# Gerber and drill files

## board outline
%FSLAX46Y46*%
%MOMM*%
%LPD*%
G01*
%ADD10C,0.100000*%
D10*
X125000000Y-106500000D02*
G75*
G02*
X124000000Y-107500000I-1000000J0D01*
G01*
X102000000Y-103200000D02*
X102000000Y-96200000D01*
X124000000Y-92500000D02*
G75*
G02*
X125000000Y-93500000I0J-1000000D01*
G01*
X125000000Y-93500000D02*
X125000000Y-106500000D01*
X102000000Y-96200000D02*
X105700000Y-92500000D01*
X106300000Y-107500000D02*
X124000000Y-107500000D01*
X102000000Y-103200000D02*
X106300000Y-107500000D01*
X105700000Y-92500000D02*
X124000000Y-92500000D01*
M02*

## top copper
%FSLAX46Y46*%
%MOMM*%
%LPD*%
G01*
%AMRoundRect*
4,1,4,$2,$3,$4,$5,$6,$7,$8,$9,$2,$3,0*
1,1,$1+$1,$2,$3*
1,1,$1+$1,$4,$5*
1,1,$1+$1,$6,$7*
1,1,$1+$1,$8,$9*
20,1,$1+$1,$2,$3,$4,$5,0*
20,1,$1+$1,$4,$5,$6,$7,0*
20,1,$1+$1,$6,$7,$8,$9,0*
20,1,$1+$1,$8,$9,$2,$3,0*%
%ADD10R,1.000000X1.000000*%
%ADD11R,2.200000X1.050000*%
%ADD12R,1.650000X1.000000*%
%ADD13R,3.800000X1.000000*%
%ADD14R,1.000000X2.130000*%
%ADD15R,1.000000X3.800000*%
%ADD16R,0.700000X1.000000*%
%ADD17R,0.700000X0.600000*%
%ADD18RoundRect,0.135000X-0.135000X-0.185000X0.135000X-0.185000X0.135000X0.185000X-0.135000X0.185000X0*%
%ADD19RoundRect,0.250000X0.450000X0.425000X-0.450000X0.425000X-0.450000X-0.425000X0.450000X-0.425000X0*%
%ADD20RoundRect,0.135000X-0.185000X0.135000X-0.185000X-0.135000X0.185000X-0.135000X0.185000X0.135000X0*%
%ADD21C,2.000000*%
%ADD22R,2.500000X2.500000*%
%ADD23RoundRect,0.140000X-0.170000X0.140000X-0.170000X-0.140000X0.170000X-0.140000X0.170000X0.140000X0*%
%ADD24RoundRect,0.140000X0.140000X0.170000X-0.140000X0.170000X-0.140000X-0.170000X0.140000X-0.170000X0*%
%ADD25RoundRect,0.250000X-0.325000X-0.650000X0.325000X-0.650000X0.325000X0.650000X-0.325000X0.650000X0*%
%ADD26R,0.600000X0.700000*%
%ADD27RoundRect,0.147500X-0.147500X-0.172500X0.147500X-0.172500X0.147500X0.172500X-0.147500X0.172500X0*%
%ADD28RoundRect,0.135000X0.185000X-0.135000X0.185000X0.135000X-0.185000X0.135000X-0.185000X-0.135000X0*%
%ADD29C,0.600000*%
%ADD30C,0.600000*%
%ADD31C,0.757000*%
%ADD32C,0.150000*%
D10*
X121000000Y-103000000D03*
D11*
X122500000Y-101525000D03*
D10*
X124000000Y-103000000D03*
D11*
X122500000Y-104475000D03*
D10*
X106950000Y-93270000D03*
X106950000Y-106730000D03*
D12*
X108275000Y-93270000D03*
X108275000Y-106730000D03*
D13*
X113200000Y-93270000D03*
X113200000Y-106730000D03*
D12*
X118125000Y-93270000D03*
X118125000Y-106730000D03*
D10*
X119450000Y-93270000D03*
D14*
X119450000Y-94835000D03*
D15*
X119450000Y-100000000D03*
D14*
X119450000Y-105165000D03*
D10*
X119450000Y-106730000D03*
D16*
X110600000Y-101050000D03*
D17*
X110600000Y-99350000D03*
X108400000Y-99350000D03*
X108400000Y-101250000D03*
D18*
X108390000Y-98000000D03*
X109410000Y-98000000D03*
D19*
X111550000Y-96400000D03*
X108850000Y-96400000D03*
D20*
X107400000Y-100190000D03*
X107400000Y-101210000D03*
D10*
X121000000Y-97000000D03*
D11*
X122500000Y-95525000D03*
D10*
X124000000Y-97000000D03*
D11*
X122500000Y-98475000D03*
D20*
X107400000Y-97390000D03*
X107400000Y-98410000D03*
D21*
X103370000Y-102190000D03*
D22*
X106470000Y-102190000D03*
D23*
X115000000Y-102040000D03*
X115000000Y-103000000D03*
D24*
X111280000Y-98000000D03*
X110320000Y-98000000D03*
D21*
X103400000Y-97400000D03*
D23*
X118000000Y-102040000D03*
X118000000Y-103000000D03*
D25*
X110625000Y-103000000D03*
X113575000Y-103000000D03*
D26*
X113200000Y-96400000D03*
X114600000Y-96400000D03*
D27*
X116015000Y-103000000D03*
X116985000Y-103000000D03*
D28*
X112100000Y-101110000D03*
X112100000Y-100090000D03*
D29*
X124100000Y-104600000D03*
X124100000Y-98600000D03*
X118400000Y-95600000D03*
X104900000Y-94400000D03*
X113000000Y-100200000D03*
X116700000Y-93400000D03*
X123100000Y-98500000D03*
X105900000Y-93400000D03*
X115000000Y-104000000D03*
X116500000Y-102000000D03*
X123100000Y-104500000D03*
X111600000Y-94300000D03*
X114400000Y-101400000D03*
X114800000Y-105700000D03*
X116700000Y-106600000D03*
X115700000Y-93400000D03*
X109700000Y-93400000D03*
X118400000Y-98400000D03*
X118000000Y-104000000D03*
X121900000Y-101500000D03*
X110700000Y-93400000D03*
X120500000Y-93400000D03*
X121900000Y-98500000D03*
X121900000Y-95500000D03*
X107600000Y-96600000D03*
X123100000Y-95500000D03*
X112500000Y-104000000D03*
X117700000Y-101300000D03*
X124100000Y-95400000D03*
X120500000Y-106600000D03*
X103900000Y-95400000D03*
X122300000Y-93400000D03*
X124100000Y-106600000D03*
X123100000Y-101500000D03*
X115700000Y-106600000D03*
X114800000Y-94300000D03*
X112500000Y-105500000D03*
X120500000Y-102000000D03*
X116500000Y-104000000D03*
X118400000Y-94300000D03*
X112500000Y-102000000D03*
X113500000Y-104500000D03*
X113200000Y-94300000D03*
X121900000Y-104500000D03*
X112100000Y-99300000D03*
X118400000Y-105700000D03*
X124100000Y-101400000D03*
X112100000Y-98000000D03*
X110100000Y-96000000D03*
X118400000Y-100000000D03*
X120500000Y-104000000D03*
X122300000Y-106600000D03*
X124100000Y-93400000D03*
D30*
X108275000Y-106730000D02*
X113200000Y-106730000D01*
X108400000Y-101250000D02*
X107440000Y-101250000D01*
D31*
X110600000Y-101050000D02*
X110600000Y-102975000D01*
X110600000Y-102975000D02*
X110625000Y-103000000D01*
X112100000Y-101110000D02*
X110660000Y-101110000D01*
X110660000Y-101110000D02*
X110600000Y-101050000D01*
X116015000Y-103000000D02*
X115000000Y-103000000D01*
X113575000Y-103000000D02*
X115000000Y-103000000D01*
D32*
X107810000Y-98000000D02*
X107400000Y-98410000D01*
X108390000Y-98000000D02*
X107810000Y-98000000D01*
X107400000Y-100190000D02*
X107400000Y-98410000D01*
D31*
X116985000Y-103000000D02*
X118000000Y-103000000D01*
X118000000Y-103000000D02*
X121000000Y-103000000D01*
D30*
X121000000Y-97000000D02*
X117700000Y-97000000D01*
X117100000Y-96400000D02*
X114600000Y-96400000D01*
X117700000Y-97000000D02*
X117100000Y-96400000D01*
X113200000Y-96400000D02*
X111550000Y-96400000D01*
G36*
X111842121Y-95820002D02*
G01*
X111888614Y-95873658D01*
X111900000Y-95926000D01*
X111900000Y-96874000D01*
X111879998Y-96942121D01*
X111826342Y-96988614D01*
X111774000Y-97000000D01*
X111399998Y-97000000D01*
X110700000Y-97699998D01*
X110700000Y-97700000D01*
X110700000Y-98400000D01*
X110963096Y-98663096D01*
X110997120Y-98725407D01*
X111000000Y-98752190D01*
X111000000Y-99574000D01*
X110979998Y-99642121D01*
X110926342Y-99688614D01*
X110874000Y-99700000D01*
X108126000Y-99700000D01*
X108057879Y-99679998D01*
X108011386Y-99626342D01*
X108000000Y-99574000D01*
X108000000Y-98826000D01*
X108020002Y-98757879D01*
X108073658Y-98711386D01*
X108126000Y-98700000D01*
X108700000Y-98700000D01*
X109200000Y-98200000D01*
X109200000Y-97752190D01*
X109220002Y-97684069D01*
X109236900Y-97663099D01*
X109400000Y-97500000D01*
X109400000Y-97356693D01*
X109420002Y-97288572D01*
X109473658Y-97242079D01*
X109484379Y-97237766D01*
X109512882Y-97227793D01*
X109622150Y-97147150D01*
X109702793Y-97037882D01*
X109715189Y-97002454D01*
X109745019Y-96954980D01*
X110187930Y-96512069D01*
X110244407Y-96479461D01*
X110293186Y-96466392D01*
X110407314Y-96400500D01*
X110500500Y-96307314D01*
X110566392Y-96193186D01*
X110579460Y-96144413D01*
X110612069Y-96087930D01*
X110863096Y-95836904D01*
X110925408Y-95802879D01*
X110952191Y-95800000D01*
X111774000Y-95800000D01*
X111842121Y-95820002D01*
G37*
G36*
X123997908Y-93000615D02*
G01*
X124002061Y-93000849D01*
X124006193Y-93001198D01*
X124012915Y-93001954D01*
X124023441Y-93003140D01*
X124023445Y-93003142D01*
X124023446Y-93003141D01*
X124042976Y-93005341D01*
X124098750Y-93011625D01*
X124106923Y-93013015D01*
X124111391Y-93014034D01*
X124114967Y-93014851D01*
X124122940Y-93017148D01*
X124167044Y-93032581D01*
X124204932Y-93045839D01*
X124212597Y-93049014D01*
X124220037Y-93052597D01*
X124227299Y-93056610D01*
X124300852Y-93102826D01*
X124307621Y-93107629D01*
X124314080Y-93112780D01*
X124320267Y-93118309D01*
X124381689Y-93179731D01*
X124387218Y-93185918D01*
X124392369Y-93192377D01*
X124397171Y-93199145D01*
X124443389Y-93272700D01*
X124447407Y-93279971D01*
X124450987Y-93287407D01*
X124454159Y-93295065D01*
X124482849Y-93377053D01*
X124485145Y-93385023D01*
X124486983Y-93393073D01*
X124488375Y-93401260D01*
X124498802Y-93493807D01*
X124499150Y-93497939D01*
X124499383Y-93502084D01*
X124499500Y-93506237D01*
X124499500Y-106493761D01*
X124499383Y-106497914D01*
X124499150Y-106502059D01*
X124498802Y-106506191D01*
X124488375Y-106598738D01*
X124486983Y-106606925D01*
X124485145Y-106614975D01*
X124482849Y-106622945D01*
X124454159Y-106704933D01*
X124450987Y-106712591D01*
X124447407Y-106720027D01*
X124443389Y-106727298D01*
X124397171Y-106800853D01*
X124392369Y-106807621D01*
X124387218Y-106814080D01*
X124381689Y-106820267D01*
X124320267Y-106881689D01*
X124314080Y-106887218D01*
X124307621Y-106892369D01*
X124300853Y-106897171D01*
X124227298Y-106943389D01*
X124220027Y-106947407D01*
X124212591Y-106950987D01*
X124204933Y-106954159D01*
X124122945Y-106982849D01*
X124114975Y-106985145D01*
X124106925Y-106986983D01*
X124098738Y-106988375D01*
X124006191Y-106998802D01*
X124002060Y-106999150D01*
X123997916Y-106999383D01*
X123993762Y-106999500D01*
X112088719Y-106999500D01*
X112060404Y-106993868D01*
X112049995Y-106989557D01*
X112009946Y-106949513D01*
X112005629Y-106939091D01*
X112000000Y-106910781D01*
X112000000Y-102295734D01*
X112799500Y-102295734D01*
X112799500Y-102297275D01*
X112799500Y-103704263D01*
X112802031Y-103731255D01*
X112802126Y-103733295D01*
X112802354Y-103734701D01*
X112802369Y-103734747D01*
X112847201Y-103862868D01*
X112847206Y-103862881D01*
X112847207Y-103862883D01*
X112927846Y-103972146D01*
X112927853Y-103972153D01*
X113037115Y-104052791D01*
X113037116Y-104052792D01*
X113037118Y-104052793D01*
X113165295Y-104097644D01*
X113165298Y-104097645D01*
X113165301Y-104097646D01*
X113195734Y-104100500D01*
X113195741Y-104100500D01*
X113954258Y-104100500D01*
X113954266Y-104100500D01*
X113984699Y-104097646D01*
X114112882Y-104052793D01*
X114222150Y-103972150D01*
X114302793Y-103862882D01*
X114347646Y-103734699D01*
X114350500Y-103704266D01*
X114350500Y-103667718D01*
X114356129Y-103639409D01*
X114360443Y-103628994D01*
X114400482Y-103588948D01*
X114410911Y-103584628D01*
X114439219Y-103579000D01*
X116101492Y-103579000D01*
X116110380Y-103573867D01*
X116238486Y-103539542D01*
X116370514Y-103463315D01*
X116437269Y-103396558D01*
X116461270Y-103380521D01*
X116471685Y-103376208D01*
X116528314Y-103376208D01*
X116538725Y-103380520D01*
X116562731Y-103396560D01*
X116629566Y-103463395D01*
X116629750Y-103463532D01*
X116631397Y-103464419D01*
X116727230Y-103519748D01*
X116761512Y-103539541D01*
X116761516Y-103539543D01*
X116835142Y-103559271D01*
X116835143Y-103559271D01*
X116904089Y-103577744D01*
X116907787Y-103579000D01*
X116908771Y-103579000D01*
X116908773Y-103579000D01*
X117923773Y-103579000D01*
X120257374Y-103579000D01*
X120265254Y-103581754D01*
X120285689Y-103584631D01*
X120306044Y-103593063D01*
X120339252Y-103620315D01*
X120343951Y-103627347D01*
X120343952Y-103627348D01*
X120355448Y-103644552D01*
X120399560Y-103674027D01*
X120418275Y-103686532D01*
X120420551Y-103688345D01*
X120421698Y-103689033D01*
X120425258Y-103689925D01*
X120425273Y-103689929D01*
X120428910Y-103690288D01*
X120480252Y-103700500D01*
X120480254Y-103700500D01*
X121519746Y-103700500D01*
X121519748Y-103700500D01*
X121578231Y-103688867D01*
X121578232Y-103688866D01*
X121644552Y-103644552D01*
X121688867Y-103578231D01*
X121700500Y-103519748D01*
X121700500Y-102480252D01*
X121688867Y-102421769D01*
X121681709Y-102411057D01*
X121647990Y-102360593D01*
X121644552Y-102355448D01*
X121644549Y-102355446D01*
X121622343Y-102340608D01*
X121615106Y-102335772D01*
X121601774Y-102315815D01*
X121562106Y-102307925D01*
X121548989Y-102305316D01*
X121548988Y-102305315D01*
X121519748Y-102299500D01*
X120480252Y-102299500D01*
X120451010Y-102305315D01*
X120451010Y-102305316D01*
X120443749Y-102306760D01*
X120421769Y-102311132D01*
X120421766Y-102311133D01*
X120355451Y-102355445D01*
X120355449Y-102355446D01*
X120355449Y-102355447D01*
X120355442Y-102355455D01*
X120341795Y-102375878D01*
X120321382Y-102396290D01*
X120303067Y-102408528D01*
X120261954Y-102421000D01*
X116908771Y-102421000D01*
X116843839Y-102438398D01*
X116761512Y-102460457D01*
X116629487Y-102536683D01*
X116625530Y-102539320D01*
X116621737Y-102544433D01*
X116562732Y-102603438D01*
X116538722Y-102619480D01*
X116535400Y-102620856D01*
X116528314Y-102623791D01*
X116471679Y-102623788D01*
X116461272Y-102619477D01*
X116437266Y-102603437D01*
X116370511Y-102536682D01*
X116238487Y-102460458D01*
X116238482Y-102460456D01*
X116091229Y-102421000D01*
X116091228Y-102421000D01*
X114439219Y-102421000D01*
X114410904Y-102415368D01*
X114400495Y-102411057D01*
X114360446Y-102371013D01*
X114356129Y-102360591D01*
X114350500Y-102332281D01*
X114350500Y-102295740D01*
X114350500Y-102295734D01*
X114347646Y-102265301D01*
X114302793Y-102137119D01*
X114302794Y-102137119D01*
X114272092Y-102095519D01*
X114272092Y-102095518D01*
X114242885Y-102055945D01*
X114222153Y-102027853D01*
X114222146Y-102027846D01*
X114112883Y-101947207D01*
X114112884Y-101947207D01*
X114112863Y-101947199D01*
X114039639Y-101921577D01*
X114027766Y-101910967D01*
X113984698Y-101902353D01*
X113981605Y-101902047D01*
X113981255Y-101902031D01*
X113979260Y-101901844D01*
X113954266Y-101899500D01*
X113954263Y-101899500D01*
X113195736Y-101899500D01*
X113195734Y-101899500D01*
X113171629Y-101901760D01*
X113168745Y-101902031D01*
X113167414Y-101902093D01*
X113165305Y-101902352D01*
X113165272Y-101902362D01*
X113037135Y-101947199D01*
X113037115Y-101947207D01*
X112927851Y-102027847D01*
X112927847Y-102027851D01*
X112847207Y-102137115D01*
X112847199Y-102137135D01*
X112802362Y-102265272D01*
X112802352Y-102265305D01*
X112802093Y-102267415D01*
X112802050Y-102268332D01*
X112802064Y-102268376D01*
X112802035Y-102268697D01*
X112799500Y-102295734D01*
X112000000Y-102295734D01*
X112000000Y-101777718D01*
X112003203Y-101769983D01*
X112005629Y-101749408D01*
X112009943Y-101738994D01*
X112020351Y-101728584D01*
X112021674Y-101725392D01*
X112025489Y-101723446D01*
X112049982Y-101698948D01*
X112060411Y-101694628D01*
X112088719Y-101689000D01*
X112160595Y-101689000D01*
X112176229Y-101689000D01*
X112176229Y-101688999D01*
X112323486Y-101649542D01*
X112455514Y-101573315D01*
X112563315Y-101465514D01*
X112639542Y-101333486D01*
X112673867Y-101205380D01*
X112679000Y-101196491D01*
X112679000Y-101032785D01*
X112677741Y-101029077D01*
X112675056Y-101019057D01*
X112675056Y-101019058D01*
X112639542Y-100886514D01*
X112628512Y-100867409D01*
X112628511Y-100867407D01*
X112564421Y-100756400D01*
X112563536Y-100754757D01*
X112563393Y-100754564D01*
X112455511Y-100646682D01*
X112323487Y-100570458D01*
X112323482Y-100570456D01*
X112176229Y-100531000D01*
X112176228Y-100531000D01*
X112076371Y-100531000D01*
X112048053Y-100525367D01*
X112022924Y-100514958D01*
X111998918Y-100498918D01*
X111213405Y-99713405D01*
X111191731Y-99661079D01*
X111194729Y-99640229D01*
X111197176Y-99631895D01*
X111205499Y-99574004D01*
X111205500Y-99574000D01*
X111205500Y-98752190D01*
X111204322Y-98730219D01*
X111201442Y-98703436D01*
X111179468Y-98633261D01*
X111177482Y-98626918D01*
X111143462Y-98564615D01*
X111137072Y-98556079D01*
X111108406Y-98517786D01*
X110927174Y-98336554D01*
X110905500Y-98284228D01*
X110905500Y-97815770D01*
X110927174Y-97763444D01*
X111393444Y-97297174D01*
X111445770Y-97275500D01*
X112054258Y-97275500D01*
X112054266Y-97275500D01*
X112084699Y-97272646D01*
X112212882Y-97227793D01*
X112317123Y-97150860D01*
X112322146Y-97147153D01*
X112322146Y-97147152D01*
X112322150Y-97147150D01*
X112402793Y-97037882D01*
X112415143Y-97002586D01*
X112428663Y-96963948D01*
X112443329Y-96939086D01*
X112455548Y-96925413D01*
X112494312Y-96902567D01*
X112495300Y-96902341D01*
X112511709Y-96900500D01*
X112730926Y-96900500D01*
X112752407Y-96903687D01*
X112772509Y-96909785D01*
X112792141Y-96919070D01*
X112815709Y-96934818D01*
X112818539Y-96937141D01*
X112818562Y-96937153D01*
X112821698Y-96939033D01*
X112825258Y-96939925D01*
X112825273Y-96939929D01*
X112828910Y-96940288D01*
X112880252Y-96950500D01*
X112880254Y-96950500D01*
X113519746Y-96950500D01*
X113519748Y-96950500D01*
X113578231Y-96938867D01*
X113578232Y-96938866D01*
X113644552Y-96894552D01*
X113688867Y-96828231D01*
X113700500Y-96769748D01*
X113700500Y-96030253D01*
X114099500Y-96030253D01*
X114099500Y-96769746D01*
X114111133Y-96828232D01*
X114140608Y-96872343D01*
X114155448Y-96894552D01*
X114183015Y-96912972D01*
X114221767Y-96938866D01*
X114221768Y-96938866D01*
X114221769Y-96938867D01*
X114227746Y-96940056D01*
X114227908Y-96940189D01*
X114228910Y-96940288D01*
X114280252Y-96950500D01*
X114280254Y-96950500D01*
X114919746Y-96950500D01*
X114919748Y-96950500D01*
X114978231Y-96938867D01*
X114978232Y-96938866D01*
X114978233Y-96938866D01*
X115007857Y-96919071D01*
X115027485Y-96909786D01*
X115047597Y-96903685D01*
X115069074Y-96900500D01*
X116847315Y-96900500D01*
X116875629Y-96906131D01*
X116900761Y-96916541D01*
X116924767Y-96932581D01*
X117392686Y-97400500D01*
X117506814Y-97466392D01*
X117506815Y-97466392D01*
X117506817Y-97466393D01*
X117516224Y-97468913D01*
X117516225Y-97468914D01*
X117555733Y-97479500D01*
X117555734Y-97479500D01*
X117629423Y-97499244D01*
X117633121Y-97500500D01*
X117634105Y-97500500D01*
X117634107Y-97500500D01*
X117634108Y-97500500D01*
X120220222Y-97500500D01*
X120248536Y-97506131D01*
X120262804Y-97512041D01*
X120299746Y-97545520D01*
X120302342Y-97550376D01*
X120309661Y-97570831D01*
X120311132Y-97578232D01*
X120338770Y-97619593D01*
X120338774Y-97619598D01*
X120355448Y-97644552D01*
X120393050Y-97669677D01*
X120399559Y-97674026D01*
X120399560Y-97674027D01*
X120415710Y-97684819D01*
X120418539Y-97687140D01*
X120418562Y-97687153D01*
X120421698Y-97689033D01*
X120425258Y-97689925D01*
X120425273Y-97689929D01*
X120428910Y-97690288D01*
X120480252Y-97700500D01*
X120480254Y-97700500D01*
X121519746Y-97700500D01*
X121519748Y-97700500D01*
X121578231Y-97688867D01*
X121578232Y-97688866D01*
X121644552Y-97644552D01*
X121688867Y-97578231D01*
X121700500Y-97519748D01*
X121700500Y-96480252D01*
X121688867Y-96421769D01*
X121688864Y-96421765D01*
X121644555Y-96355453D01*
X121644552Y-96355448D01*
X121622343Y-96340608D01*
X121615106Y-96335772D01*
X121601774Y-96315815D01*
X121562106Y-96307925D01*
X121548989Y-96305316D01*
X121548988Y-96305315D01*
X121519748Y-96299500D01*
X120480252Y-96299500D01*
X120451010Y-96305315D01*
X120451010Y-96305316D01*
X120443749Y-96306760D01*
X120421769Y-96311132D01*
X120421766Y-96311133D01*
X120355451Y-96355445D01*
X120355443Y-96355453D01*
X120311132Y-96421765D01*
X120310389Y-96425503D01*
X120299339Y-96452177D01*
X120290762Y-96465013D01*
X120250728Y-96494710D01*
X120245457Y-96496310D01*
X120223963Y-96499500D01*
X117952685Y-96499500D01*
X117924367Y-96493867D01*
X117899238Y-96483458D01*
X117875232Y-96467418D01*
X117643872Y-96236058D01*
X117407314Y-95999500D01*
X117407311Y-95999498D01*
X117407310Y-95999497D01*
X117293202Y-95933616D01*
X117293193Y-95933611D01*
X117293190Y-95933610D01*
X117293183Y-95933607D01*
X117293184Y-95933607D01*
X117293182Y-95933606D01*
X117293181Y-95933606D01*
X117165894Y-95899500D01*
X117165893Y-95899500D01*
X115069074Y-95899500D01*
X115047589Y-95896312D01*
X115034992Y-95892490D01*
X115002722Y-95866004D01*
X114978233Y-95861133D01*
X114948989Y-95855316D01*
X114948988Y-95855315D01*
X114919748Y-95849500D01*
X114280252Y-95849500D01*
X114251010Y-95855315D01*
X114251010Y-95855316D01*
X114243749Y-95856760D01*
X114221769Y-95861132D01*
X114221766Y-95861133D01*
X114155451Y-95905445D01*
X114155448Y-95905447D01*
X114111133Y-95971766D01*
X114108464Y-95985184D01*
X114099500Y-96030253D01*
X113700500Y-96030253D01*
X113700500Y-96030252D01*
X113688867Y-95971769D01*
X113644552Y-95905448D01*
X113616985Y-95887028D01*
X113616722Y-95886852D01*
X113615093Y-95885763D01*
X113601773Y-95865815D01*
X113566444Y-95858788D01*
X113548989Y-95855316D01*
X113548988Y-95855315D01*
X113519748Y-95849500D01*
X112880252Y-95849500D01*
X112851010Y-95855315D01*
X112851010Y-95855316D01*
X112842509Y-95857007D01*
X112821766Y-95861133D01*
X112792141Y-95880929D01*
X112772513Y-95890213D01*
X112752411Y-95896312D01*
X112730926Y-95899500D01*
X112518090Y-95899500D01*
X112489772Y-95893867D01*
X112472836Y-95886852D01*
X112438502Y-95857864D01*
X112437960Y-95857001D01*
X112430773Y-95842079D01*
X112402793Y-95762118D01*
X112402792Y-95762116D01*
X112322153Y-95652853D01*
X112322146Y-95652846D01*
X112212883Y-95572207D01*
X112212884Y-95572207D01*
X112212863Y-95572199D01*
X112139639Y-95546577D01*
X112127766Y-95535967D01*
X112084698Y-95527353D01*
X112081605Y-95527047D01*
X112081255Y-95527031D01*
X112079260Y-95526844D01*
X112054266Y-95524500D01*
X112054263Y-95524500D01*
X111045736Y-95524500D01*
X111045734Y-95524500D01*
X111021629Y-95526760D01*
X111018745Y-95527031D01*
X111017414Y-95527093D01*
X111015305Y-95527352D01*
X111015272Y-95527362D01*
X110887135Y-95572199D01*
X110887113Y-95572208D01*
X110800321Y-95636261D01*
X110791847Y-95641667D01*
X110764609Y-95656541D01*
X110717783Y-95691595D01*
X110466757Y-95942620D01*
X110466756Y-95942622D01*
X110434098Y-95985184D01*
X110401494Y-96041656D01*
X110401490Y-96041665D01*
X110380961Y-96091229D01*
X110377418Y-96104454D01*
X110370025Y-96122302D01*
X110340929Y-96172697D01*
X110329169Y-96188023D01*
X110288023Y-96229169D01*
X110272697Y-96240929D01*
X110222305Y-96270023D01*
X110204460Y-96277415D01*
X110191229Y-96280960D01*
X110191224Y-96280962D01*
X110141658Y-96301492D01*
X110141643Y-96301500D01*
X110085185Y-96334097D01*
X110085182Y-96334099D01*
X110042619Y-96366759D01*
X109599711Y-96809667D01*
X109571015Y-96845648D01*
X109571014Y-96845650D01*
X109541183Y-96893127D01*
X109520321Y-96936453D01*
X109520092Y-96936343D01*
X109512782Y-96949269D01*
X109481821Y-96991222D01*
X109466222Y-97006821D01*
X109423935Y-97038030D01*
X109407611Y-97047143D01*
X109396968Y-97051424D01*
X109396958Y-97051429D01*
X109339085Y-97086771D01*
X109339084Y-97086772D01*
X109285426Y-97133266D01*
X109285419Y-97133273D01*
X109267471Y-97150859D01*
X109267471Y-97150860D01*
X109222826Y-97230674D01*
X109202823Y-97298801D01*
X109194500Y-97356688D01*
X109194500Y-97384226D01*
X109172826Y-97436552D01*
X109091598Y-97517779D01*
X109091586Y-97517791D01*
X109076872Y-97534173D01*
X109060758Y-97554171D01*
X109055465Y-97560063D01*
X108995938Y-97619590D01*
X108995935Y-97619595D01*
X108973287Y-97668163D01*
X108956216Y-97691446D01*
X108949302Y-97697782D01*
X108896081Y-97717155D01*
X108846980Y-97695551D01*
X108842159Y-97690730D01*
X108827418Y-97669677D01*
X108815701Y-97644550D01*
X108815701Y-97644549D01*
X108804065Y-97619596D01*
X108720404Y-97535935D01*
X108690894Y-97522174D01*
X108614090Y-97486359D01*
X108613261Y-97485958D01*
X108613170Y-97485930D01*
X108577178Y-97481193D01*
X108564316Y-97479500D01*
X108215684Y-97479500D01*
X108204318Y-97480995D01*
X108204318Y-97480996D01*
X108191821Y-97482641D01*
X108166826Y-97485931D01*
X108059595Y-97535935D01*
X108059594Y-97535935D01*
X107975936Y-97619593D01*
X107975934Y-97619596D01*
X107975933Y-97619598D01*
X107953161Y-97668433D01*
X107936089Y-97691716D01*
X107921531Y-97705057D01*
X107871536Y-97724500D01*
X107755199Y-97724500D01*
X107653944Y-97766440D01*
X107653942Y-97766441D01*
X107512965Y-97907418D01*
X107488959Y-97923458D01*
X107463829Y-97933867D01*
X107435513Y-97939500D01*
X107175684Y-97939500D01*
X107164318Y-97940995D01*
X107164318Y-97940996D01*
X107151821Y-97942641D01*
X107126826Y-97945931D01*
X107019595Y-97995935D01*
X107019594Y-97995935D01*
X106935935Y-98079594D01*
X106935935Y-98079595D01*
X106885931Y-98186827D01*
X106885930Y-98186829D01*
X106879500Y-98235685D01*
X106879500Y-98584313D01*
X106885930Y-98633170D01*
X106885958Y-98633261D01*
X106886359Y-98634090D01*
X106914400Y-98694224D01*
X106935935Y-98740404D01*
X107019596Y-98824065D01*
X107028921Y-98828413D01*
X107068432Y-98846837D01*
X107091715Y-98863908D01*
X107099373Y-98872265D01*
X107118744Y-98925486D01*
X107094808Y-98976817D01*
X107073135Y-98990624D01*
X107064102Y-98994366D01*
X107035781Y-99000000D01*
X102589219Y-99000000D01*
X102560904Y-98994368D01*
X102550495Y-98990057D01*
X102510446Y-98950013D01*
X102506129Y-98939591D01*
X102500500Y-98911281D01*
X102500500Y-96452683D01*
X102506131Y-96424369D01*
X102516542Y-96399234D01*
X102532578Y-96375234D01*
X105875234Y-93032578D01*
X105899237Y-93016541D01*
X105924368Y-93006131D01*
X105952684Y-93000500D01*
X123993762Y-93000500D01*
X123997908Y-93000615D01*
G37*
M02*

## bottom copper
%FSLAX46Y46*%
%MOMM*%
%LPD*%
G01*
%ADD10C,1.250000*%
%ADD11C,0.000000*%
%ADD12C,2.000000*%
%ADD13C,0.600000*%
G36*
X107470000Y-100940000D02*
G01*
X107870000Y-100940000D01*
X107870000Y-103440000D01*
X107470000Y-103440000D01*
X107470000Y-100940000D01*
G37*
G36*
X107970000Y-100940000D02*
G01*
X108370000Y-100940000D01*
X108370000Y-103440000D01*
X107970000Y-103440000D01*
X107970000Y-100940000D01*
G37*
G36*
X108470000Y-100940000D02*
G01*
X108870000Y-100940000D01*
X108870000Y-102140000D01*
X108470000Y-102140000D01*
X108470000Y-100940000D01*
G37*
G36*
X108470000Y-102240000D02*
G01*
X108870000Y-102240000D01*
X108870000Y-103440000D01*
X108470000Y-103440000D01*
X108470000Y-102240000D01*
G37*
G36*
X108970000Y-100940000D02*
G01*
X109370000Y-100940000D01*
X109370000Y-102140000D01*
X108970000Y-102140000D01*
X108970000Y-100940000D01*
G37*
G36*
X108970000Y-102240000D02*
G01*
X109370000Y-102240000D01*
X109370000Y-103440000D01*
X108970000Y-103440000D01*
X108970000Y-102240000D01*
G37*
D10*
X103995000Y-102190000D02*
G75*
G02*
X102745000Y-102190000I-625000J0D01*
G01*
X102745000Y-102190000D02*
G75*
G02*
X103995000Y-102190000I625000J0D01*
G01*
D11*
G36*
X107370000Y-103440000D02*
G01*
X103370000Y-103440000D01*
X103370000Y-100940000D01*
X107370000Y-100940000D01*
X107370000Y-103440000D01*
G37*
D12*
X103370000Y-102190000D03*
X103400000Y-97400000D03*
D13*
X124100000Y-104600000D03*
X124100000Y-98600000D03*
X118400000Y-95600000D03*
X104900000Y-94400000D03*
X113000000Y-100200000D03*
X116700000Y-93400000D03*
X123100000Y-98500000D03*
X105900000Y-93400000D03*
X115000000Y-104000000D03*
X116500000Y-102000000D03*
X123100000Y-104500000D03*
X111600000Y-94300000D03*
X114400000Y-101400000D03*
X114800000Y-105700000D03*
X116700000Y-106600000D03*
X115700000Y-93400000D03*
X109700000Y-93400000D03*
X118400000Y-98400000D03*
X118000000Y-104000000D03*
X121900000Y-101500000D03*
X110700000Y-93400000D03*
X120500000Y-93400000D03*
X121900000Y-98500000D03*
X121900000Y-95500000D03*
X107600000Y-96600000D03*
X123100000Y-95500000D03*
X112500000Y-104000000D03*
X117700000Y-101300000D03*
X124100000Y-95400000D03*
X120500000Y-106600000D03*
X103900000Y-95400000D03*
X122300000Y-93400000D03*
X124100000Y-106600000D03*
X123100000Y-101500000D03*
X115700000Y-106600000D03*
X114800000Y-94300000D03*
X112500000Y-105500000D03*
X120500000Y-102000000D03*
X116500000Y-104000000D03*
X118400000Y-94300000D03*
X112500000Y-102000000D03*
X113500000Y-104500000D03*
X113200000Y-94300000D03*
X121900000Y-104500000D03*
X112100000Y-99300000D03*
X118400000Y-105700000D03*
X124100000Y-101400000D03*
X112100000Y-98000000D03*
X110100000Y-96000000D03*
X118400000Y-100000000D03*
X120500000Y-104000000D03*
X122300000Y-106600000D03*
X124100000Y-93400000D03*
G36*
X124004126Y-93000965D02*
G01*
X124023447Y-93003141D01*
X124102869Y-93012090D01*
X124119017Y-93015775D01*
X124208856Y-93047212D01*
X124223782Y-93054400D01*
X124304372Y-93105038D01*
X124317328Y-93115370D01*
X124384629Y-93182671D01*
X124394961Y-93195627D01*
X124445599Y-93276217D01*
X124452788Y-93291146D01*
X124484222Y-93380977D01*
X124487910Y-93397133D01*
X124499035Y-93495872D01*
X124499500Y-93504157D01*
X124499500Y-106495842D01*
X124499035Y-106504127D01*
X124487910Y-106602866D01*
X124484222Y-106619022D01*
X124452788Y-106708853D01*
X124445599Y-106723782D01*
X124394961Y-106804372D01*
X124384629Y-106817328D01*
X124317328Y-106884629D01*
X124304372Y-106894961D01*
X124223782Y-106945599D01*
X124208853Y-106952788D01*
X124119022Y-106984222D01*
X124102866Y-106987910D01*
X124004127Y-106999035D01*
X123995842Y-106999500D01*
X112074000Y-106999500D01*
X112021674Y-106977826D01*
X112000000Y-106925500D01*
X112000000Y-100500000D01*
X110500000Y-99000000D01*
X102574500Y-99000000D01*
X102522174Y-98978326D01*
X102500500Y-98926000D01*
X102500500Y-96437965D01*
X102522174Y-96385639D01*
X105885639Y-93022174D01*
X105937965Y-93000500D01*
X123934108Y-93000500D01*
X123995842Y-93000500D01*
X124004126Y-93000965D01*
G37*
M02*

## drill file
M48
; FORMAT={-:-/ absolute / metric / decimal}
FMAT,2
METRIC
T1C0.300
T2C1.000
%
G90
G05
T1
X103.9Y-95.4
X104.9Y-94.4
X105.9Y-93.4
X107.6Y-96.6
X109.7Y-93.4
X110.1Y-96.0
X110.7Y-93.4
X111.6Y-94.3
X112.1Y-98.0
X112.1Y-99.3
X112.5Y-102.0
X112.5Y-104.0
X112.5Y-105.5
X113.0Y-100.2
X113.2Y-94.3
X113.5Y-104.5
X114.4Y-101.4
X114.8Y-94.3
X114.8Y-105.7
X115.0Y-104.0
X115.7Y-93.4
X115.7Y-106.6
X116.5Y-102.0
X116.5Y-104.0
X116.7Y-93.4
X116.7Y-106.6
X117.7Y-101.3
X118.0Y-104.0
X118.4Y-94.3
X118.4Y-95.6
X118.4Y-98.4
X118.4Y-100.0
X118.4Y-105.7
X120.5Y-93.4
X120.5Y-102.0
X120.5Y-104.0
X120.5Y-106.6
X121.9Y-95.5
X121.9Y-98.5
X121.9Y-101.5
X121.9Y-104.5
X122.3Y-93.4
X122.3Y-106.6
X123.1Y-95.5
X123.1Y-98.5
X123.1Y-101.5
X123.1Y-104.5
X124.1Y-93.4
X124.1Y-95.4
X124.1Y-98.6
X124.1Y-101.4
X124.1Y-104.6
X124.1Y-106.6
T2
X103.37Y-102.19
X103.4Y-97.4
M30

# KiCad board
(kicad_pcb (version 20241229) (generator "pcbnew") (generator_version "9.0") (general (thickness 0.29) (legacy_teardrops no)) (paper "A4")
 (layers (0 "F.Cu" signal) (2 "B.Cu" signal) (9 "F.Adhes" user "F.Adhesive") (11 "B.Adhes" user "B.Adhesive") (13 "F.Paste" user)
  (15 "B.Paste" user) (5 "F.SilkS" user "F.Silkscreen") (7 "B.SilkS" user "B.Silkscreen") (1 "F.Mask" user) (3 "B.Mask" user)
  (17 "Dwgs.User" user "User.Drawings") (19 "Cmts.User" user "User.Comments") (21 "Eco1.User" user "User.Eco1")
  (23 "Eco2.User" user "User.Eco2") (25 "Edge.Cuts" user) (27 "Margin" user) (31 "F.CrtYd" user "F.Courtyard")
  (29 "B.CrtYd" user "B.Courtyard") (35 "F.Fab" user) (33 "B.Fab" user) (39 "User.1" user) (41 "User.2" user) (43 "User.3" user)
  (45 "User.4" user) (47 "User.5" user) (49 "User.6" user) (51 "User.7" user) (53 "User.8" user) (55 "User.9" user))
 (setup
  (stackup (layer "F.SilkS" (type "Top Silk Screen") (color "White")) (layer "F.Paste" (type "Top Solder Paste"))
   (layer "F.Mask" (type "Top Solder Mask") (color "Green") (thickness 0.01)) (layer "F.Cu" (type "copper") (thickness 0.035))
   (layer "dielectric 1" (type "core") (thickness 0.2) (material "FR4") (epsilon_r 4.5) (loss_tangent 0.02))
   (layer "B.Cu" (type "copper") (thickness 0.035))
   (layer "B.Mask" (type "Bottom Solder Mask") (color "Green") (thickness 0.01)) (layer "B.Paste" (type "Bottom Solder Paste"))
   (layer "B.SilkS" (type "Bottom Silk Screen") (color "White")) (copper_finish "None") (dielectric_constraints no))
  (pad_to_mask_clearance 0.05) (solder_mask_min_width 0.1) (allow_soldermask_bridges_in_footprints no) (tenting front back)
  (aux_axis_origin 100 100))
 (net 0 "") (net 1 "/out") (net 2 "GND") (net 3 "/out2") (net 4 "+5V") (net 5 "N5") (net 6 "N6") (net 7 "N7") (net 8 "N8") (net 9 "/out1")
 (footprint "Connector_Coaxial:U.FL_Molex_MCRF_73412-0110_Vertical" (layer "F.Cu") (at 122.5 103 -90)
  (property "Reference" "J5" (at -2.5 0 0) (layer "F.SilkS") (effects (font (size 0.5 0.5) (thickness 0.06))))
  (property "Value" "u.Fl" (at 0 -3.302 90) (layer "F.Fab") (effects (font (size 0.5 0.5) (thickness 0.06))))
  (pad "1" smd rect (at 0 1.5 270) (size 1 1) (layers "F.Cu" "F.Mask" "F.Paste") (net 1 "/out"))
  (pad "2" smd rect (at -1.475 0 270) (size 1.05 2.2) (layers "F.Cu" "F.Mask" "F.Paste") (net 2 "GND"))
  (pad "2" smd rect (at 0 -1.5 270) (size 1 1) (layers "F.Cu" "F.Mask" "F.Paste") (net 2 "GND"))
  (pad "2" smd rect (at 1.475 0 270) (size 1.05 2.2) (layers "F.Cu" "F.Mask" "F.Paste") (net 2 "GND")))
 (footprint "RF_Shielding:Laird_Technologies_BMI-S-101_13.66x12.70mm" (layer "F.Cu") (at 113.2 100)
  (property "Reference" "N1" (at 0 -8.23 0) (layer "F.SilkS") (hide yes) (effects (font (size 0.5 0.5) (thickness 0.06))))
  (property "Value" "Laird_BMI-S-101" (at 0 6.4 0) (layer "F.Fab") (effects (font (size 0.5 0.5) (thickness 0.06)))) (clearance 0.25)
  (pad "1" smd rect (at -6.25 -6.73) (size 1 1) (layers "F.Cu" "F.Mask" "F.Paste") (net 2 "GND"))
  (pad "1" smd rect (at -6.25 6.73) (size 1 1) (layers "F.Cu" "F.Mask" "F.Paste") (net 2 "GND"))
  (pad "1" smd rect (at -4.925 -6.73) (size 1.65 1) (layers "F.Cu" "F.Mask" "F.Paste") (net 2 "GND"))
  (pad "1" smd rect (at -4.925 6.73) (size 1.65 1) (layers "F.Cu" "F.Mask" "F.Paste") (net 2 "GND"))
  (pad "1" smd rect (at 0 -6.73) (size 3.8 1) (layers "F.Cu" "F.Mask" "F.Paste") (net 2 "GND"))
  (pad "1" smd rect (at 0 6.73) (size 3.8 1) (layers "F.Cu" "F.Mask" "F.Paste") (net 2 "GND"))
  (pad "1" smd rect (at 4.925 -6.73) (size 1.65 1) (layers "F.Cu" "F.Mask" "F.Paste") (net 2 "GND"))
  (pad "1" smd rect (at 4.925 6.73) (size 1.65 1) (layers "F.Cu" "F.Mask" "F.Paste") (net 2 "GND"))
  (pad "1" smd rect (at 6.25 -6.73) (size 1 1) (layers "F.Cu" "F.Mask" "F.Paste") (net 2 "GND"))
  (pad "1" smd rect (at 6.25 -5.165) (size 1 2.13) (layers "F.Cu" "F.Mask" "F.Paste") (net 2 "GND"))
  (pad "1" smd rect (at 6.25 0) (size 1 3.8) (layers "F.Cu" "F.Mask" "F.Paste") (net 2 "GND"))
  (pad "1" smd rect (at 6.25 5.165) (size 1 2.13) (layers "F.Cu" "F.Mask" "F.Paste") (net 2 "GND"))
  (pad "1" smd rect (at 6.25 6.73) (size 1 1) (layers "F.Cu" "F.Mask" "F.Paste") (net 2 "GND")))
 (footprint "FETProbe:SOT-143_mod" (layer "F.Cu") (at 109.5 100.3 180)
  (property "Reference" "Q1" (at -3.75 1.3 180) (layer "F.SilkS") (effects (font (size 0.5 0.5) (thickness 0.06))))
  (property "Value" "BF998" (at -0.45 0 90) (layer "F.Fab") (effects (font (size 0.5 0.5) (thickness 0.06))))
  (pad "1" smd rect (at -1.1 -0.75 180) (size 0.7 1) (layers "F.Cu" "F.Mask" "F.Paste") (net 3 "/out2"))
  (pad "2" smd rect (at -1.1 0.95 180) (size 0.7 0.6) (layers "F.Cu" "F.Mask" "F.Paste") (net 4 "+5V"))
  (pad "3" smd rect (at 1.1 0.95 180) (size 0.7 0.6) (layers "F.Cu" "F.Mask" "F.Paste") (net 4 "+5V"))
  (pad "4" smd rect (at 1.1 -0.95 180) (size 0.7 0.6) (layers "F.Cu" "F.Mask" "F.Paste") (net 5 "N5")))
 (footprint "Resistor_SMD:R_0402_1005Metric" (layer "F.Cu") (at 108.9 98)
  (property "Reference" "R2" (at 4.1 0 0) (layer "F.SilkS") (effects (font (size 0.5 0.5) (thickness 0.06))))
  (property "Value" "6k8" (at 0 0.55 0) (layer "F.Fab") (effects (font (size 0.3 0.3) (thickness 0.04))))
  (pad "1" smd roundrect (at -0.51 0) (size 0.54 0.64) (layers "F.Cu" "F.Mask" "F.Paste") (roundrect_rratio 0.25) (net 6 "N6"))
  (pad "2" smd roundrect (at 0.51 0) (size 0.54 0.64) (layers "F.Cu" "F.Mask" "F.Paste") (roundrect_rratio 0.25) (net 4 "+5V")))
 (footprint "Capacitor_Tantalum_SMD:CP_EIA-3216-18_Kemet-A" (layer "F.Cu") (at 110.2 96.4 180)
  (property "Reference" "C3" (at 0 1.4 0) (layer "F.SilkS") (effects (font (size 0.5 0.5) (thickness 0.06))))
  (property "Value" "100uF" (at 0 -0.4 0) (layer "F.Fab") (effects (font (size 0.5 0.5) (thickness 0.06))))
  (pad "1" smd roundrect (at -1.35 0 180) (size 1.4 1.35) (layers "F.Cu" "F.Mask" "F.Paste") (roundrect_rratio 0.1851851852) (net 4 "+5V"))
  (pad "2" smd roundrect (at 1.35 0 180) (size 1.4 1.35) (layers "F.Cu" "F.Mask" "F.Paste") (roundrect_rratio 0.1851851852) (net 2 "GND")))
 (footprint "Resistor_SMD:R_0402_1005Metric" (layer "F.Cu") (at 107.4 100.7 -90)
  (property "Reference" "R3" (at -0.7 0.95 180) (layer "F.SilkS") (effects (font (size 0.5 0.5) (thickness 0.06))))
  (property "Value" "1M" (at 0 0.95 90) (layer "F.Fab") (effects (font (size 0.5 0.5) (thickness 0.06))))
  (pad "1" smd roundrect (at -0.51 0 270) (size 0.54 0.64) (layers "F.Cu" "F.Mask" "F.Paste") (roundrect_rratio 0.25) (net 6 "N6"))
  (pad "2" smd roundrect (at 0.51 0 270) (size 0.54 0.64) (layers "F.Cu" "F.Mask" "F.Paste") (roundrect_rratio 0.25) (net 5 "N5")))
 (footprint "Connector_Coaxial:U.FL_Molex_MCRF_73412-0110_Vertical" (layer "F.Cu") (at 122.5 97 -90)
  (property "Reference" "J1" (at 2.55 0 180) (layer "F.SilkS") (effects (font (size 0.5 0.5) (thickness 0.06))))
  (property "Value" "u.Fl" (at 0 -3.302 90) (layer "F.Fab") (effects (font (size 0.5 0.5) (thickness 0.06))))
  (pad "1" smd rect (at 0 1.5 270) (size 1 1) (layers "F.Cu" "F.Mask" "F.Paste") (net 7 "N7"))
  (pad "2" smd rect (at -1.475 0 270) (size 1.05 2.2) (layers "F.Cu" "F.Mask" "F.Paste") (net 2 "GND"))
  (pad "2" smd rect (at 0 -1.5 270) (size 1 1) (layers "F.Cu" "F.Mask" "F.Paste") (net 2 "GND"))
  (pad "2" smd rect (at 1.475 0 270) (size 1.05 2.2) (layers "F.Cu" "F.Mask" "F.Paste") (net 2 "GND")))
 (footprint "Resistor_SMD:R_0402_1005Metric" (layer "F.Cu") (at 107.4 97.9 -90)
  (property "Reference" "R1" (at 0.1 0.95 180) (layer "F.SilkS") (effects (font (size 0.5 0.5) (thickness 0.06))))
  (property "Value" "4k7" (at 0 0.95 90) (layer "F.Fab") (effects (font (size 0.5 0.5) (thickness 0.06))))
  (pad "1" smd roundrect (at -0.51 0 270) (size 0.54 0.64) (layers "F.Cu" "F.Mask" "F.Paste") (roundrect_rratio 0.25) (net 2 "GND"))
  (pad "2" smd roundrect (at 0.51 0 270) (size 0.54 0.64) (layers "F.Cu" "F.Mask" "F.Paste") (roundrect_rratio 0.25) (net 6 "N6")))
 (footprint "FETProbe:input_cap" (layer "F.Cu") (at 108.07 102.19)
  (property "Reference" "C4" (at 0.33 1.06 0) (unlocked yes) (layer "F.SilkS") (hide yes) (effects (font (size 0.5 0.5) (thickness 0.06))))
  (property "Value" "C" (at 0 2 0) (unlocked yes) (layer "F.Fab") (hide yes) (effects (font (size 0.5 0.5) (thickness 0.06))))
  (fp_rect (start -0.6 -1.25) (end -0.2 1.25) (stroke (width 0) (type solid)) (fill yes) (layer "B.Cu"))
  (fp_rect (start -0.1 -1.25) (end 0.3 1.25) (stroke (width 0) (type solid)) (fill yes) (layer "B.Cu"))
  (fp_rect (start 0.4 -1.25) (end 0.8 -0.05) (stroke (width 0) (type solid)) (fill yes) (layer "B.Cu"))
  (fp_rect (start 0.4 0.05) (end 0.8 1.25) (stroke (width 0) (type solid)) (fill yes) (layer "B.Cu"))
  (fp_rect (start 0.9 -1.25) (end 1.3 -0.05) (stroke (width 0) (type solid)) (fill yes) (layer "B.Cu"))
  (fp_rect (start 0.9 0.05) (end 1.3 1.25) (stroke (width 0) (type solid)) (fill yes) (layer "B.Cu"))
  (fp_circle (center -4.7 0) (end -3.45 0) (stroke (width 0) (type solid)) (fill yes) (layer "B.Cu"))
  (fp_poly (pts (xy -4.7 -1.25) (xy -0.7 -1.25) (xy -0.7 1.25) (xy -4.7 1.25)) (stroke (width 0) (type solid)) (fill yes) (layer "B.Cu"))
  (pad "1" thru_hole circle (at -4.7 0) (size 2 2) (drill 1) (layers "*.Cu" "*.Mask") (remove_unused_layers no) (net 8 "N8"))
  (pad "2" smd rect (at -1.6 0) (size 2.5 2.5) (layers "F.Cu") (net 5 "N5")))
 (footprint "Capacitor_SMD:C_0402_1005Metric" (layer "F.Cu") (at 115 102.52 -90)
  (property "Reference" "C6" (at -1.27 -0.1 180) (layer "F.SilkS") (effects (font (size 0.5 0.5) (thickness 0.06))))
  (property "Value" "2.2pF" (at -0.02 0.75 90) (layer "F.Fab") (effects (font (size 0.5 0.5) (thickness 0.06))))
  (pad "1" smd roundrect (at -0.48 0 270) (size 0.56 0.62) (layers "F.Cu" "F.Mask" "F.Paste") (roundrect_rratio 0.25) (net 2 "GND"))
  (pad "2" smd roundrect (at 0.48 0 270) (size 0.56 0.62) (layers "F.Cu" "F.Mask" "F.Paste") (roundrect_rratio 0.25) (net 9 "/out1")))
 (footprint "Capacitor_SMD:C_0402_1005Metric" (layer "F.Cu") (at 110.8 98 180)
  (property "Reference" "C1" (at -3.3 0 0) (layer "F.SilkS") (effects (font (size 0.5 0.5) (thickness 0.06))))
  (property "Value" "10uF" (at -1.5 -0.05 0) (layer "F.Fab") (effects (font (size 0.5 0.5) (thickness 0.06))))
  (pad "1" smd roundrect (at -0.48 0 180) (size 0.56 0.62) (layers "F.Cu" "F.Mask" "F.Paste") (roundrect_rratio 0.25) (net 2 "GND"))
  (pad "2" smd roundrect (at 0.48 0 180) (size 0.56 0.62) (layers "F.Cu" "F.Mask" "F.Paste") (roundrect_rratio 0.25) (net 4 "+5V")))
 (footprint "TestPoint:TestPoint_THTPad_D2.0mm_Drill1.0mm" (layer "F.Cu") (at 103.4 97.4)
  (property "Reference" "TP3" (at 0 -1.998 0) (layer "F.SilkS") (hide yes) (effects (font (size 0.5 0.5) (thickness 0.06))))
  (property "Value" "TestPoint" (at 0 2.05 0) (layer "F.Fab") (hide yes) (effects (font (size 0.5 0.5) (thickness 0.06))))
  (pad "1" thru_hole circle (at 0 0) (size 2 2) (drill 1) (layers "*.Cu" "*.Mask") (remove_unused_layers no) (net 2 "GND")))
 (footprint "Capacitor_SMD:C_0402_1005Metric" (layer "F.Cu") (at 118 102.52 -90)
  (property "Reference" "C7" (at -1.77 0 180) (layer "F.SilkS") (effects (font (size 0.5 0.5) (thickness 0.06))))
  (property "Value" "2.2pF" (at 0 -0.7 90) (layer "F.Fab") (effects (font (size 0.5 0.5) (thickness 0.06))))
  (pad "1" smd roundrect (at -0.48 0 270) (size 0.56 0.62) (layers "F.Cu" "F.Mask" "F.Paste") (roundrect_rratio 0.25) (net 2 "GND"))
  (pad "2" smd roundrect (at 0.48 0 270) (size 0.56 0.62) (layers "F.Cu" "F.Mask" "F.Paste") (roundrect_rratio 0.25) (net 1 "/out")))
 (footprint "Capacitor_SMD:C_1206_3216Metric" (layer "F.Cu") (at 112.1 103)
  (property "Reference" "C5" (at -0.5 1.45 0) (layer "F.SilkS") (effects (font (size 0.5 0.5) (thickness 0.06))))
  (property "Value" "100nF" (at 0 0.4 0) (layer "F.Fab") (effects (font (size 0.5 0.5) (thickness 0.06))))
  (pad "1" smd roundrect (at -1.475 0) (size 1.15 1.8) (layers "F.Cu" "F.Mask" "F.Paste") (roundrect_rratio 0.2173913043) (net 3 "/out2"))
  (pad "2" smd roundrect (at 1.475 0) (size 1.15 1.8) (layers "F.Cu" "F.Mask" "F.Paste") (roundrect_rratio 0.2173913043) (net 9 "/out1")))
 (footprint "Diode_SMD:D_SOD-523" (layer "F.Cu") (at 113.9 96.4)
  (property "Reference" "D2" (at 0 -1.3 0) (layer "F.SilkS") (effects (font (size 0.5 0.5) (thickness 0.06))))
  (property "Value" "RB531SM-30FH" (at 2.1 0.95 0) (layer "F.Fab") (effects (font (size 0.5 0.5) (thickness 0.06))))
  (pad "1" smd rect (at -0.7 0 180) (size 0.6 0.7) (layers "F.Cu" "F.Mask" "F.Paste") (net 4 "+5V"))
  (pad "2" smd rect (at 0.7 0 180) (size 0.6 0.7) (layers "F.Cu" "F.Mask" "F.Paste") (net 7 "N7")))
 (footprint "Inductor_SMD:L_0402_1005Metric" (layer "F.Cu") (at 116.5 103)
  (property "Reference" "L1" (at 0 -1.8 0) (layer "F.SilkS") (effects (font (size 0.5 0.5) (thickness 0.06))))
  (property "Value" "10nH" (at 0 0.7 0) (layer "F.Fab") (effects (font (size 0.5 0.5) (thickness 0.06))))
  (pad "1" smd roundrect (at -0.485 0) (size 0.59 0.64) (layers "F.Cu" "F.Mask" "F.Paste") (roundrect_rratio 0.25) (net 9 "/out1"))
  (pad "2" smd roundrect (at 0.485 0) (size 0.59 0.64) (layers "F.Cu" "F.Mask" "F.Paste") (roundrect_rratio 0.25) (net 1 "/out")))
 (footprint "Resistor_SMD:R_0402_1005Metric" (layer "F.Cu") (at 112.1 100.6 90)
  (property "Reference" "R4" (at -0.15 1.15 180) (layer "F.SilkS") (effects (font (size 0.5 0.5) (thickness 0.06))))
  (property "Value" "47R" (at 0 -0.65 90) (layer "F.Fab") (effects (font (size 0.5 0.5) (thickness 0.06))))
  (pad "1" smd roundrect (at -0.51 0 90) (size 0.54 0.64) (layers "F.Cu" "F.Mask" "F.Paste") (roundrect_rratio 0.25) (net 3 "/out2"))
  (pad "2" smd roundrect (at 0.51 0 90) (size 0.54 0.64) (layers "F.Cu" "F.Mask" "F.Paste") (roundrect_rratio 0.25) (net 2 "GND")))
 (gr_arc (start 125 106.5) (mid 124.707107 107.207107) (end 124 107.5) (stroke (width 0.1) (type solid)) (layer "Edge.Cuts"))
 (gr_line (start 102 103.2) (end 102 96.2) (stroke (width 0.1) (type solid)) (layer "Edge.Cuts"))
 (gr_arc (start 124 92.5) (mid 124.707107 92.792893) (end 125 93.5) (stroke (width 0.1) (type solid)) (layer "Edge.Cuts"))
 (gr_line (start 125 93.5) (end 125 106.5) (stroke (width 0.1) (type solid)) (layer "Edge.Cuts"))
 (gr_line (start 102 96.2) (end 105.7 92.5) (stroke (width 0.1) (type solid)) (layer "Edge.Cuts"))
 (gr_line (start 106.3 107.5) (end 124 107.5) (stroke (width 0.1) (type solid)) (layer "Edge.Cuts"))
 (gr_line (start 102 103.2) (end 106.3 107.5) (stroke (width 0.1) (type solid)) (layer "Edge.Cuts"))
 (gr_line (start 105.7 92.5) (end 124 92.5) (stroke (width 0.1) (type solid)) (layer "Edge.Cuts"))
 (segment (start 108.275 106.73) (end 113.2 106.73) (width 0.6) (layer "F.Cu") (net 2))
 (via (at 124.1 104.6) (size 0.6) (drill 0.3) (layers "F.Cu" "B.Cu") (free yes) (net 2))
 (via (at 124.1 98.6) (size 0.6) (drill 0.3) (layers "F.Cu" "B.Cu") (free yes) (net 2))
 (via (at 118.4 95.6) (size 0.6) (drill 0.3) (layers "F.Cu" "B.Cu") (free yes) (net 2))
 (via (at 104.9 94.4) (size 0.6) (drill 0.3) (layers "F.Cu" "B.Cu") (free yes) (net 2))
 (via (at 113 100.2) (size 0.6) (drill 0.3) (layers "F.Cu" "B.Cu") (free yes) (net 2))
 (via (at 116.7 93.4) (size 0.6) (drill 0.3) (layers "F.Cu" "B.Cu") (free yes) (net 2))
 (via (at 123.1 98.5) (size 0.6) (drill 0.3) (layers "F.Cu" "B.Cu") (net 2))
 (via (at 105.9 93.4) (size 0.6) (drill 0.3) (layers "F.Cu" "B.Cu") (free yes) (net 2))
 (via (at 115 104) (size 0.6) (drill 0.3) (layers "F.Cu" "B.Cu") (free yes) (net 2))
 (via (at 116.5 102) (size 0.6) (drill 0.3) (layers "F.Cu" "B.Cu") (free yes) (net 2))
 (via (at 123.1 104.5) (size 0.6) (drill 0.3) (layers "F.Cu" "B.Cu") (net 2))
 (via (at 111.6 94.3) (size 0.6) (drill 0.3) (layers "F.Cu" "B.Cu") (free yes) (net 2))
 (via (at 114.4 101.4) (size 0.6) (drill 0.3) (layers "F.Cu" "B.Cu") (free yes) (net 2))
 (via (at 114.8 105.7) (size 0.6) (drill 0.3) (layers "F.Cu" "B.Cu") (free yes) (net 2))
 (via (at 116.7 106.6) (size 0.6) (drill 0.3) (layers "F.Cu" "B.Cu") (free yes) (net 2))
 (via (at 115.7 93.4) (size 0.6) (drill 0.3) (layers "F.Cu" "B.Cu") (free yes) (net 2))
 (via (at 109.7 93.4) (size 0.6) (drill 0.3) (layers "F.Cu" "B.Cu") (free yes) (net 2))
 (via (at 118.4 98.4) (size 0.6) (drill 0.3) (layers "F.Cu" "B.Cu") (free yes) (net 2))
 (via (at 118 104) (size 0.6) (drill 0.3) (layers "F.Cu" "B.Cu") (free yes) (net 2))
 (via (at 121.9 101.5) (size 0.6) (drill 0.3) (layers "F.Cu" "B.Cu") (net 2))
 (via (at 110.7 93.4) (size 0.6) (drill 0.3) (layers "F.Cu" "B.Cu") (free yes) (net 2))
 (via (at 120.5 93.4) (size 0.6) (drill 0.3) (layers "F.Cu" "B.Cu") (free yes) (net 2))
 (via (at 121.9 98.5) (size 0.6) (drill 0.3) (layers "F.Cu" "B.Cu") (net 2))
 (via (at 121.9 95.5) (size 0.6) (drill 0.3) (layers "F.Cu" "B.Cu") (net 2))
 (via (at 107.6 96.6) (size 0.6) (drill 0.3) (layers "F.Cu" "B.Cu") (free yes) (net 2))
 (via (at 123.1 95.5) (size 0.6) (drill 0.3) (layers "F.Cu" "B.Cu") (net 2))
 (via (at 112.5 104) (size 0.6) (drill 0.3) (layers "F.Cu" "B.Cu") (free yes) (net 2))
 (via (at 117.7 101.3) (size 0.6) (drill 0.3) (layers "F.Cu" "B.Cu") (free yes) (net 2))
 (via (at 124.1 95.4) (size 0.6) (drill 0.3) (layers "F.Cu" "B.Cu") (free yes) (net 2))
 (via (at 120.5 106.6) (size 0.6) (drill 0.3) (layers "F.Cu" "B.Cu") (free yes) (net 2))
 (via (at 103.9 95.4) (size 0.6) (drill 0.3) (layers "F.Cu" "B.Cu") (free yes) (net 2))
 (via (at 122.3 93.4) (size 0.6) (drill 0.3) (layers "F.Cu" "B.Cu") (free yes) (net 2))
 (via (at 124.1 106.6) (size 0.6) (drill 0.3) (layers "F.Cu" "B.Cu") (free yes) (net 2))
 (via (at 123.1 101.5) (size 0.6) (drill 0.3) (layers "F.Cu" "B.Cu") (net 2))
 (via (at 115.7 106.6) (size 0.6) (drill 0.3) (layers "F.Cu" "B.Cu") (free yes) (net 2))
 (via (at 114.8 94.3) (size 0.6) (drill 0.3) (layers "F.Cu" "B.Cu") (free yes) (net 2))
 (via (at 112.5 105.5) (size 0.6) (drill 0.3) (layers "F.Cu" "B.Cu") (free yes) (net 2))
 (via (at 120.5 102) (size 0.6) (drill 0.3) (layers "F.Cu" "B.Cu") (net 2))
 (via (at 116.5 104) (size 0.6) (drill 0.3) (layers "F.Cu" "B.Cu") (free yes) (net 2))
 (via (at 118.4 94.3) (size 0.6) (drill 0.3) (layers "F.Cu" "B.Cu") (free yes) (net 2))
 (via (at 112.5 102) (size 0.6) (drill 0.3) (layers "F.Cu" "B.Cu") (free yes) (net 2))
 (via (at 113.5 104.5) (size 0.6) (drill 0.3) (layers "F.Cu" "B.Cu") (free yes) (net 2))
 (via (at 113.2 94.3) (size 0.6) (drill 0.3) (layers "F.Cu" "B.Cu") (free yes) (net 2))
 (via (at 121.9 104.5) (size 0.6) (drill 0.3) (layers "F.Cu" "B.Cu") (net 2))
 (via (at 112.1 99.3) (size 0.6) (drill 0.3) (layers "F.Cu" "B.Cu") (free yes) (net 2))
 (via (at 118.4 105.7) (size 0.6) (drill 0.3) (layers "F.Cu" "B.Cu") (free yes) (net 2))
 (via (at 124.1 101.4) (size 0.6) (drill 0.3) (layers "F.Cu" "B.Cu") (free yes) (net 2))
 (via (at 112.1 98) (size 0.6) (drill 0.3) (layers "F.Cu" "B.Cu") (free yes) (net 2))
 (via (at 110.1 96) (size 0.6) (drill 0.3) (layers "F.Cu" "B.Cu") (free yes) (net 2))
 (via (at 118.4 100) (size 0.6) (drill 0.3) (layers "F.Cu" "B.Cu") (free yes) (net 2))
 (via (at 120.5 104) (size 0.6) (drill 0.3) (layers "F.Cu" "B.Cu") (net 2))
 (via (at 122.3 106.6) (size 0.6) (drill 0.3) (layers "F.Cu" "B.Cu") (free yes) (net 2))
 (via (at 124.1 93.4) (size 0.6) (drill 0.3) (layers "F.Cu" "B.Cu") (free yes) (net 2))
 (segment (start 108.4 101.25) (end 107.44 101.25) (width 0.6) (layer "F.Cu") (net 5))
 (segment (start 110.6 101.05) (end 110.6 102.975) (width 0.757) (layer "F.Cu") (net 3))
 (segment (start 110.6 102.975) (end 110.625 103) (width 0.757) (layer "F.Cu") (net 3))
 (segment (start 112.1 101.11) (end 110.66 101.11) (width 0.757) (layer "F.Cu") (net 3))
 (segment (start 110.66 101.11) (end 110.6 101.05) (width 0.757) (layer "F.Cu") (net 3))
 (segment (start 116.015 103) (end 115 103) (width 0.757) (layer "F.Cu") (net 9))
 (segment (start 113.575 103) (end 115 103) (width 0.757) (layer "F.Cu") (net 9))
 (segment (start 107.81 98) (end 107.4 98.41) (width 0.15) (layer "F.Cu") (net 6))
 (segment (start 108.39 98) (end 107.81 98) (width 0.15) (layer "F.Cu") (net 6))
 (segment (start 107.4 100.19) (end 107.4 98.41) (width 0.15) (layer "F.Cu") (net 6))
 (segment (start 116.985 103) (end 118 103) (width 0.757) (layer "F.Cu") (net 1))
 (segment (start 118 103) (end 121 103) (width 0.757) (layer "F.Cu") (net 1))
 (segment (start 121 97) (end 117.7 97) (width 0.6) (layer "F.Cu") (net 7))
 (segment (start 117.1 96.4) (end 114.6 96.4) (width 0.6) (layer "F.Cu") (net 7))
 (segment (start 117.7 97) (end 117.1 96.4) (width 0.6) (layer "F.Cu") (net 7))
 (segment (start 113.2 96.4) (end 111.55 96.4) (width 0.6) (layer "F.Cu") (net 4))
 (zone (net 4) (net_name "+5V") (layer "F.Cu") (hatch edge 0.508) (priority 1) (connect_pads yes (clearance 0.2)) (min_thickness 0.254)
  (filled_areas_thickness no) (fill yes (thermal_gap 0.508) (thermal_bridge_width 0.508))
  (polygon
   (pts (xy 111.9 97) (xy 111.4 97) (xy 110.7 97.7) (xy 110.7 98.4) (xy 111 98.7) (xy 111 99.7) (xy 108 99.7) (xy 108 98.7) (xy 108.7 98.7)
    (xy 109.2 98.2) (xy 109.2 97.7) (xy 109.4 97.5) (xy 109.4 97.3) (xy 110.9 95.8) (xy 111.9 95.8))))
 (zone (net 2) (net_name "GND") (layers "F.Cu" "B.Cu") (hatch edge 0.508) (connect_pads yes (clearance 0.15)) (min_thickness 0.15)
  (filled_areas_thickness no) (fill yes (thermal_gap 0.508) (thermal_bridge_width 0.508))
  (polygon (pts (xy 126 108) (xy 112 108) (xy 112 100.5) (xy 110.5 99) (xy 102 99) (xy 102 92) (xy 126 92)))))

